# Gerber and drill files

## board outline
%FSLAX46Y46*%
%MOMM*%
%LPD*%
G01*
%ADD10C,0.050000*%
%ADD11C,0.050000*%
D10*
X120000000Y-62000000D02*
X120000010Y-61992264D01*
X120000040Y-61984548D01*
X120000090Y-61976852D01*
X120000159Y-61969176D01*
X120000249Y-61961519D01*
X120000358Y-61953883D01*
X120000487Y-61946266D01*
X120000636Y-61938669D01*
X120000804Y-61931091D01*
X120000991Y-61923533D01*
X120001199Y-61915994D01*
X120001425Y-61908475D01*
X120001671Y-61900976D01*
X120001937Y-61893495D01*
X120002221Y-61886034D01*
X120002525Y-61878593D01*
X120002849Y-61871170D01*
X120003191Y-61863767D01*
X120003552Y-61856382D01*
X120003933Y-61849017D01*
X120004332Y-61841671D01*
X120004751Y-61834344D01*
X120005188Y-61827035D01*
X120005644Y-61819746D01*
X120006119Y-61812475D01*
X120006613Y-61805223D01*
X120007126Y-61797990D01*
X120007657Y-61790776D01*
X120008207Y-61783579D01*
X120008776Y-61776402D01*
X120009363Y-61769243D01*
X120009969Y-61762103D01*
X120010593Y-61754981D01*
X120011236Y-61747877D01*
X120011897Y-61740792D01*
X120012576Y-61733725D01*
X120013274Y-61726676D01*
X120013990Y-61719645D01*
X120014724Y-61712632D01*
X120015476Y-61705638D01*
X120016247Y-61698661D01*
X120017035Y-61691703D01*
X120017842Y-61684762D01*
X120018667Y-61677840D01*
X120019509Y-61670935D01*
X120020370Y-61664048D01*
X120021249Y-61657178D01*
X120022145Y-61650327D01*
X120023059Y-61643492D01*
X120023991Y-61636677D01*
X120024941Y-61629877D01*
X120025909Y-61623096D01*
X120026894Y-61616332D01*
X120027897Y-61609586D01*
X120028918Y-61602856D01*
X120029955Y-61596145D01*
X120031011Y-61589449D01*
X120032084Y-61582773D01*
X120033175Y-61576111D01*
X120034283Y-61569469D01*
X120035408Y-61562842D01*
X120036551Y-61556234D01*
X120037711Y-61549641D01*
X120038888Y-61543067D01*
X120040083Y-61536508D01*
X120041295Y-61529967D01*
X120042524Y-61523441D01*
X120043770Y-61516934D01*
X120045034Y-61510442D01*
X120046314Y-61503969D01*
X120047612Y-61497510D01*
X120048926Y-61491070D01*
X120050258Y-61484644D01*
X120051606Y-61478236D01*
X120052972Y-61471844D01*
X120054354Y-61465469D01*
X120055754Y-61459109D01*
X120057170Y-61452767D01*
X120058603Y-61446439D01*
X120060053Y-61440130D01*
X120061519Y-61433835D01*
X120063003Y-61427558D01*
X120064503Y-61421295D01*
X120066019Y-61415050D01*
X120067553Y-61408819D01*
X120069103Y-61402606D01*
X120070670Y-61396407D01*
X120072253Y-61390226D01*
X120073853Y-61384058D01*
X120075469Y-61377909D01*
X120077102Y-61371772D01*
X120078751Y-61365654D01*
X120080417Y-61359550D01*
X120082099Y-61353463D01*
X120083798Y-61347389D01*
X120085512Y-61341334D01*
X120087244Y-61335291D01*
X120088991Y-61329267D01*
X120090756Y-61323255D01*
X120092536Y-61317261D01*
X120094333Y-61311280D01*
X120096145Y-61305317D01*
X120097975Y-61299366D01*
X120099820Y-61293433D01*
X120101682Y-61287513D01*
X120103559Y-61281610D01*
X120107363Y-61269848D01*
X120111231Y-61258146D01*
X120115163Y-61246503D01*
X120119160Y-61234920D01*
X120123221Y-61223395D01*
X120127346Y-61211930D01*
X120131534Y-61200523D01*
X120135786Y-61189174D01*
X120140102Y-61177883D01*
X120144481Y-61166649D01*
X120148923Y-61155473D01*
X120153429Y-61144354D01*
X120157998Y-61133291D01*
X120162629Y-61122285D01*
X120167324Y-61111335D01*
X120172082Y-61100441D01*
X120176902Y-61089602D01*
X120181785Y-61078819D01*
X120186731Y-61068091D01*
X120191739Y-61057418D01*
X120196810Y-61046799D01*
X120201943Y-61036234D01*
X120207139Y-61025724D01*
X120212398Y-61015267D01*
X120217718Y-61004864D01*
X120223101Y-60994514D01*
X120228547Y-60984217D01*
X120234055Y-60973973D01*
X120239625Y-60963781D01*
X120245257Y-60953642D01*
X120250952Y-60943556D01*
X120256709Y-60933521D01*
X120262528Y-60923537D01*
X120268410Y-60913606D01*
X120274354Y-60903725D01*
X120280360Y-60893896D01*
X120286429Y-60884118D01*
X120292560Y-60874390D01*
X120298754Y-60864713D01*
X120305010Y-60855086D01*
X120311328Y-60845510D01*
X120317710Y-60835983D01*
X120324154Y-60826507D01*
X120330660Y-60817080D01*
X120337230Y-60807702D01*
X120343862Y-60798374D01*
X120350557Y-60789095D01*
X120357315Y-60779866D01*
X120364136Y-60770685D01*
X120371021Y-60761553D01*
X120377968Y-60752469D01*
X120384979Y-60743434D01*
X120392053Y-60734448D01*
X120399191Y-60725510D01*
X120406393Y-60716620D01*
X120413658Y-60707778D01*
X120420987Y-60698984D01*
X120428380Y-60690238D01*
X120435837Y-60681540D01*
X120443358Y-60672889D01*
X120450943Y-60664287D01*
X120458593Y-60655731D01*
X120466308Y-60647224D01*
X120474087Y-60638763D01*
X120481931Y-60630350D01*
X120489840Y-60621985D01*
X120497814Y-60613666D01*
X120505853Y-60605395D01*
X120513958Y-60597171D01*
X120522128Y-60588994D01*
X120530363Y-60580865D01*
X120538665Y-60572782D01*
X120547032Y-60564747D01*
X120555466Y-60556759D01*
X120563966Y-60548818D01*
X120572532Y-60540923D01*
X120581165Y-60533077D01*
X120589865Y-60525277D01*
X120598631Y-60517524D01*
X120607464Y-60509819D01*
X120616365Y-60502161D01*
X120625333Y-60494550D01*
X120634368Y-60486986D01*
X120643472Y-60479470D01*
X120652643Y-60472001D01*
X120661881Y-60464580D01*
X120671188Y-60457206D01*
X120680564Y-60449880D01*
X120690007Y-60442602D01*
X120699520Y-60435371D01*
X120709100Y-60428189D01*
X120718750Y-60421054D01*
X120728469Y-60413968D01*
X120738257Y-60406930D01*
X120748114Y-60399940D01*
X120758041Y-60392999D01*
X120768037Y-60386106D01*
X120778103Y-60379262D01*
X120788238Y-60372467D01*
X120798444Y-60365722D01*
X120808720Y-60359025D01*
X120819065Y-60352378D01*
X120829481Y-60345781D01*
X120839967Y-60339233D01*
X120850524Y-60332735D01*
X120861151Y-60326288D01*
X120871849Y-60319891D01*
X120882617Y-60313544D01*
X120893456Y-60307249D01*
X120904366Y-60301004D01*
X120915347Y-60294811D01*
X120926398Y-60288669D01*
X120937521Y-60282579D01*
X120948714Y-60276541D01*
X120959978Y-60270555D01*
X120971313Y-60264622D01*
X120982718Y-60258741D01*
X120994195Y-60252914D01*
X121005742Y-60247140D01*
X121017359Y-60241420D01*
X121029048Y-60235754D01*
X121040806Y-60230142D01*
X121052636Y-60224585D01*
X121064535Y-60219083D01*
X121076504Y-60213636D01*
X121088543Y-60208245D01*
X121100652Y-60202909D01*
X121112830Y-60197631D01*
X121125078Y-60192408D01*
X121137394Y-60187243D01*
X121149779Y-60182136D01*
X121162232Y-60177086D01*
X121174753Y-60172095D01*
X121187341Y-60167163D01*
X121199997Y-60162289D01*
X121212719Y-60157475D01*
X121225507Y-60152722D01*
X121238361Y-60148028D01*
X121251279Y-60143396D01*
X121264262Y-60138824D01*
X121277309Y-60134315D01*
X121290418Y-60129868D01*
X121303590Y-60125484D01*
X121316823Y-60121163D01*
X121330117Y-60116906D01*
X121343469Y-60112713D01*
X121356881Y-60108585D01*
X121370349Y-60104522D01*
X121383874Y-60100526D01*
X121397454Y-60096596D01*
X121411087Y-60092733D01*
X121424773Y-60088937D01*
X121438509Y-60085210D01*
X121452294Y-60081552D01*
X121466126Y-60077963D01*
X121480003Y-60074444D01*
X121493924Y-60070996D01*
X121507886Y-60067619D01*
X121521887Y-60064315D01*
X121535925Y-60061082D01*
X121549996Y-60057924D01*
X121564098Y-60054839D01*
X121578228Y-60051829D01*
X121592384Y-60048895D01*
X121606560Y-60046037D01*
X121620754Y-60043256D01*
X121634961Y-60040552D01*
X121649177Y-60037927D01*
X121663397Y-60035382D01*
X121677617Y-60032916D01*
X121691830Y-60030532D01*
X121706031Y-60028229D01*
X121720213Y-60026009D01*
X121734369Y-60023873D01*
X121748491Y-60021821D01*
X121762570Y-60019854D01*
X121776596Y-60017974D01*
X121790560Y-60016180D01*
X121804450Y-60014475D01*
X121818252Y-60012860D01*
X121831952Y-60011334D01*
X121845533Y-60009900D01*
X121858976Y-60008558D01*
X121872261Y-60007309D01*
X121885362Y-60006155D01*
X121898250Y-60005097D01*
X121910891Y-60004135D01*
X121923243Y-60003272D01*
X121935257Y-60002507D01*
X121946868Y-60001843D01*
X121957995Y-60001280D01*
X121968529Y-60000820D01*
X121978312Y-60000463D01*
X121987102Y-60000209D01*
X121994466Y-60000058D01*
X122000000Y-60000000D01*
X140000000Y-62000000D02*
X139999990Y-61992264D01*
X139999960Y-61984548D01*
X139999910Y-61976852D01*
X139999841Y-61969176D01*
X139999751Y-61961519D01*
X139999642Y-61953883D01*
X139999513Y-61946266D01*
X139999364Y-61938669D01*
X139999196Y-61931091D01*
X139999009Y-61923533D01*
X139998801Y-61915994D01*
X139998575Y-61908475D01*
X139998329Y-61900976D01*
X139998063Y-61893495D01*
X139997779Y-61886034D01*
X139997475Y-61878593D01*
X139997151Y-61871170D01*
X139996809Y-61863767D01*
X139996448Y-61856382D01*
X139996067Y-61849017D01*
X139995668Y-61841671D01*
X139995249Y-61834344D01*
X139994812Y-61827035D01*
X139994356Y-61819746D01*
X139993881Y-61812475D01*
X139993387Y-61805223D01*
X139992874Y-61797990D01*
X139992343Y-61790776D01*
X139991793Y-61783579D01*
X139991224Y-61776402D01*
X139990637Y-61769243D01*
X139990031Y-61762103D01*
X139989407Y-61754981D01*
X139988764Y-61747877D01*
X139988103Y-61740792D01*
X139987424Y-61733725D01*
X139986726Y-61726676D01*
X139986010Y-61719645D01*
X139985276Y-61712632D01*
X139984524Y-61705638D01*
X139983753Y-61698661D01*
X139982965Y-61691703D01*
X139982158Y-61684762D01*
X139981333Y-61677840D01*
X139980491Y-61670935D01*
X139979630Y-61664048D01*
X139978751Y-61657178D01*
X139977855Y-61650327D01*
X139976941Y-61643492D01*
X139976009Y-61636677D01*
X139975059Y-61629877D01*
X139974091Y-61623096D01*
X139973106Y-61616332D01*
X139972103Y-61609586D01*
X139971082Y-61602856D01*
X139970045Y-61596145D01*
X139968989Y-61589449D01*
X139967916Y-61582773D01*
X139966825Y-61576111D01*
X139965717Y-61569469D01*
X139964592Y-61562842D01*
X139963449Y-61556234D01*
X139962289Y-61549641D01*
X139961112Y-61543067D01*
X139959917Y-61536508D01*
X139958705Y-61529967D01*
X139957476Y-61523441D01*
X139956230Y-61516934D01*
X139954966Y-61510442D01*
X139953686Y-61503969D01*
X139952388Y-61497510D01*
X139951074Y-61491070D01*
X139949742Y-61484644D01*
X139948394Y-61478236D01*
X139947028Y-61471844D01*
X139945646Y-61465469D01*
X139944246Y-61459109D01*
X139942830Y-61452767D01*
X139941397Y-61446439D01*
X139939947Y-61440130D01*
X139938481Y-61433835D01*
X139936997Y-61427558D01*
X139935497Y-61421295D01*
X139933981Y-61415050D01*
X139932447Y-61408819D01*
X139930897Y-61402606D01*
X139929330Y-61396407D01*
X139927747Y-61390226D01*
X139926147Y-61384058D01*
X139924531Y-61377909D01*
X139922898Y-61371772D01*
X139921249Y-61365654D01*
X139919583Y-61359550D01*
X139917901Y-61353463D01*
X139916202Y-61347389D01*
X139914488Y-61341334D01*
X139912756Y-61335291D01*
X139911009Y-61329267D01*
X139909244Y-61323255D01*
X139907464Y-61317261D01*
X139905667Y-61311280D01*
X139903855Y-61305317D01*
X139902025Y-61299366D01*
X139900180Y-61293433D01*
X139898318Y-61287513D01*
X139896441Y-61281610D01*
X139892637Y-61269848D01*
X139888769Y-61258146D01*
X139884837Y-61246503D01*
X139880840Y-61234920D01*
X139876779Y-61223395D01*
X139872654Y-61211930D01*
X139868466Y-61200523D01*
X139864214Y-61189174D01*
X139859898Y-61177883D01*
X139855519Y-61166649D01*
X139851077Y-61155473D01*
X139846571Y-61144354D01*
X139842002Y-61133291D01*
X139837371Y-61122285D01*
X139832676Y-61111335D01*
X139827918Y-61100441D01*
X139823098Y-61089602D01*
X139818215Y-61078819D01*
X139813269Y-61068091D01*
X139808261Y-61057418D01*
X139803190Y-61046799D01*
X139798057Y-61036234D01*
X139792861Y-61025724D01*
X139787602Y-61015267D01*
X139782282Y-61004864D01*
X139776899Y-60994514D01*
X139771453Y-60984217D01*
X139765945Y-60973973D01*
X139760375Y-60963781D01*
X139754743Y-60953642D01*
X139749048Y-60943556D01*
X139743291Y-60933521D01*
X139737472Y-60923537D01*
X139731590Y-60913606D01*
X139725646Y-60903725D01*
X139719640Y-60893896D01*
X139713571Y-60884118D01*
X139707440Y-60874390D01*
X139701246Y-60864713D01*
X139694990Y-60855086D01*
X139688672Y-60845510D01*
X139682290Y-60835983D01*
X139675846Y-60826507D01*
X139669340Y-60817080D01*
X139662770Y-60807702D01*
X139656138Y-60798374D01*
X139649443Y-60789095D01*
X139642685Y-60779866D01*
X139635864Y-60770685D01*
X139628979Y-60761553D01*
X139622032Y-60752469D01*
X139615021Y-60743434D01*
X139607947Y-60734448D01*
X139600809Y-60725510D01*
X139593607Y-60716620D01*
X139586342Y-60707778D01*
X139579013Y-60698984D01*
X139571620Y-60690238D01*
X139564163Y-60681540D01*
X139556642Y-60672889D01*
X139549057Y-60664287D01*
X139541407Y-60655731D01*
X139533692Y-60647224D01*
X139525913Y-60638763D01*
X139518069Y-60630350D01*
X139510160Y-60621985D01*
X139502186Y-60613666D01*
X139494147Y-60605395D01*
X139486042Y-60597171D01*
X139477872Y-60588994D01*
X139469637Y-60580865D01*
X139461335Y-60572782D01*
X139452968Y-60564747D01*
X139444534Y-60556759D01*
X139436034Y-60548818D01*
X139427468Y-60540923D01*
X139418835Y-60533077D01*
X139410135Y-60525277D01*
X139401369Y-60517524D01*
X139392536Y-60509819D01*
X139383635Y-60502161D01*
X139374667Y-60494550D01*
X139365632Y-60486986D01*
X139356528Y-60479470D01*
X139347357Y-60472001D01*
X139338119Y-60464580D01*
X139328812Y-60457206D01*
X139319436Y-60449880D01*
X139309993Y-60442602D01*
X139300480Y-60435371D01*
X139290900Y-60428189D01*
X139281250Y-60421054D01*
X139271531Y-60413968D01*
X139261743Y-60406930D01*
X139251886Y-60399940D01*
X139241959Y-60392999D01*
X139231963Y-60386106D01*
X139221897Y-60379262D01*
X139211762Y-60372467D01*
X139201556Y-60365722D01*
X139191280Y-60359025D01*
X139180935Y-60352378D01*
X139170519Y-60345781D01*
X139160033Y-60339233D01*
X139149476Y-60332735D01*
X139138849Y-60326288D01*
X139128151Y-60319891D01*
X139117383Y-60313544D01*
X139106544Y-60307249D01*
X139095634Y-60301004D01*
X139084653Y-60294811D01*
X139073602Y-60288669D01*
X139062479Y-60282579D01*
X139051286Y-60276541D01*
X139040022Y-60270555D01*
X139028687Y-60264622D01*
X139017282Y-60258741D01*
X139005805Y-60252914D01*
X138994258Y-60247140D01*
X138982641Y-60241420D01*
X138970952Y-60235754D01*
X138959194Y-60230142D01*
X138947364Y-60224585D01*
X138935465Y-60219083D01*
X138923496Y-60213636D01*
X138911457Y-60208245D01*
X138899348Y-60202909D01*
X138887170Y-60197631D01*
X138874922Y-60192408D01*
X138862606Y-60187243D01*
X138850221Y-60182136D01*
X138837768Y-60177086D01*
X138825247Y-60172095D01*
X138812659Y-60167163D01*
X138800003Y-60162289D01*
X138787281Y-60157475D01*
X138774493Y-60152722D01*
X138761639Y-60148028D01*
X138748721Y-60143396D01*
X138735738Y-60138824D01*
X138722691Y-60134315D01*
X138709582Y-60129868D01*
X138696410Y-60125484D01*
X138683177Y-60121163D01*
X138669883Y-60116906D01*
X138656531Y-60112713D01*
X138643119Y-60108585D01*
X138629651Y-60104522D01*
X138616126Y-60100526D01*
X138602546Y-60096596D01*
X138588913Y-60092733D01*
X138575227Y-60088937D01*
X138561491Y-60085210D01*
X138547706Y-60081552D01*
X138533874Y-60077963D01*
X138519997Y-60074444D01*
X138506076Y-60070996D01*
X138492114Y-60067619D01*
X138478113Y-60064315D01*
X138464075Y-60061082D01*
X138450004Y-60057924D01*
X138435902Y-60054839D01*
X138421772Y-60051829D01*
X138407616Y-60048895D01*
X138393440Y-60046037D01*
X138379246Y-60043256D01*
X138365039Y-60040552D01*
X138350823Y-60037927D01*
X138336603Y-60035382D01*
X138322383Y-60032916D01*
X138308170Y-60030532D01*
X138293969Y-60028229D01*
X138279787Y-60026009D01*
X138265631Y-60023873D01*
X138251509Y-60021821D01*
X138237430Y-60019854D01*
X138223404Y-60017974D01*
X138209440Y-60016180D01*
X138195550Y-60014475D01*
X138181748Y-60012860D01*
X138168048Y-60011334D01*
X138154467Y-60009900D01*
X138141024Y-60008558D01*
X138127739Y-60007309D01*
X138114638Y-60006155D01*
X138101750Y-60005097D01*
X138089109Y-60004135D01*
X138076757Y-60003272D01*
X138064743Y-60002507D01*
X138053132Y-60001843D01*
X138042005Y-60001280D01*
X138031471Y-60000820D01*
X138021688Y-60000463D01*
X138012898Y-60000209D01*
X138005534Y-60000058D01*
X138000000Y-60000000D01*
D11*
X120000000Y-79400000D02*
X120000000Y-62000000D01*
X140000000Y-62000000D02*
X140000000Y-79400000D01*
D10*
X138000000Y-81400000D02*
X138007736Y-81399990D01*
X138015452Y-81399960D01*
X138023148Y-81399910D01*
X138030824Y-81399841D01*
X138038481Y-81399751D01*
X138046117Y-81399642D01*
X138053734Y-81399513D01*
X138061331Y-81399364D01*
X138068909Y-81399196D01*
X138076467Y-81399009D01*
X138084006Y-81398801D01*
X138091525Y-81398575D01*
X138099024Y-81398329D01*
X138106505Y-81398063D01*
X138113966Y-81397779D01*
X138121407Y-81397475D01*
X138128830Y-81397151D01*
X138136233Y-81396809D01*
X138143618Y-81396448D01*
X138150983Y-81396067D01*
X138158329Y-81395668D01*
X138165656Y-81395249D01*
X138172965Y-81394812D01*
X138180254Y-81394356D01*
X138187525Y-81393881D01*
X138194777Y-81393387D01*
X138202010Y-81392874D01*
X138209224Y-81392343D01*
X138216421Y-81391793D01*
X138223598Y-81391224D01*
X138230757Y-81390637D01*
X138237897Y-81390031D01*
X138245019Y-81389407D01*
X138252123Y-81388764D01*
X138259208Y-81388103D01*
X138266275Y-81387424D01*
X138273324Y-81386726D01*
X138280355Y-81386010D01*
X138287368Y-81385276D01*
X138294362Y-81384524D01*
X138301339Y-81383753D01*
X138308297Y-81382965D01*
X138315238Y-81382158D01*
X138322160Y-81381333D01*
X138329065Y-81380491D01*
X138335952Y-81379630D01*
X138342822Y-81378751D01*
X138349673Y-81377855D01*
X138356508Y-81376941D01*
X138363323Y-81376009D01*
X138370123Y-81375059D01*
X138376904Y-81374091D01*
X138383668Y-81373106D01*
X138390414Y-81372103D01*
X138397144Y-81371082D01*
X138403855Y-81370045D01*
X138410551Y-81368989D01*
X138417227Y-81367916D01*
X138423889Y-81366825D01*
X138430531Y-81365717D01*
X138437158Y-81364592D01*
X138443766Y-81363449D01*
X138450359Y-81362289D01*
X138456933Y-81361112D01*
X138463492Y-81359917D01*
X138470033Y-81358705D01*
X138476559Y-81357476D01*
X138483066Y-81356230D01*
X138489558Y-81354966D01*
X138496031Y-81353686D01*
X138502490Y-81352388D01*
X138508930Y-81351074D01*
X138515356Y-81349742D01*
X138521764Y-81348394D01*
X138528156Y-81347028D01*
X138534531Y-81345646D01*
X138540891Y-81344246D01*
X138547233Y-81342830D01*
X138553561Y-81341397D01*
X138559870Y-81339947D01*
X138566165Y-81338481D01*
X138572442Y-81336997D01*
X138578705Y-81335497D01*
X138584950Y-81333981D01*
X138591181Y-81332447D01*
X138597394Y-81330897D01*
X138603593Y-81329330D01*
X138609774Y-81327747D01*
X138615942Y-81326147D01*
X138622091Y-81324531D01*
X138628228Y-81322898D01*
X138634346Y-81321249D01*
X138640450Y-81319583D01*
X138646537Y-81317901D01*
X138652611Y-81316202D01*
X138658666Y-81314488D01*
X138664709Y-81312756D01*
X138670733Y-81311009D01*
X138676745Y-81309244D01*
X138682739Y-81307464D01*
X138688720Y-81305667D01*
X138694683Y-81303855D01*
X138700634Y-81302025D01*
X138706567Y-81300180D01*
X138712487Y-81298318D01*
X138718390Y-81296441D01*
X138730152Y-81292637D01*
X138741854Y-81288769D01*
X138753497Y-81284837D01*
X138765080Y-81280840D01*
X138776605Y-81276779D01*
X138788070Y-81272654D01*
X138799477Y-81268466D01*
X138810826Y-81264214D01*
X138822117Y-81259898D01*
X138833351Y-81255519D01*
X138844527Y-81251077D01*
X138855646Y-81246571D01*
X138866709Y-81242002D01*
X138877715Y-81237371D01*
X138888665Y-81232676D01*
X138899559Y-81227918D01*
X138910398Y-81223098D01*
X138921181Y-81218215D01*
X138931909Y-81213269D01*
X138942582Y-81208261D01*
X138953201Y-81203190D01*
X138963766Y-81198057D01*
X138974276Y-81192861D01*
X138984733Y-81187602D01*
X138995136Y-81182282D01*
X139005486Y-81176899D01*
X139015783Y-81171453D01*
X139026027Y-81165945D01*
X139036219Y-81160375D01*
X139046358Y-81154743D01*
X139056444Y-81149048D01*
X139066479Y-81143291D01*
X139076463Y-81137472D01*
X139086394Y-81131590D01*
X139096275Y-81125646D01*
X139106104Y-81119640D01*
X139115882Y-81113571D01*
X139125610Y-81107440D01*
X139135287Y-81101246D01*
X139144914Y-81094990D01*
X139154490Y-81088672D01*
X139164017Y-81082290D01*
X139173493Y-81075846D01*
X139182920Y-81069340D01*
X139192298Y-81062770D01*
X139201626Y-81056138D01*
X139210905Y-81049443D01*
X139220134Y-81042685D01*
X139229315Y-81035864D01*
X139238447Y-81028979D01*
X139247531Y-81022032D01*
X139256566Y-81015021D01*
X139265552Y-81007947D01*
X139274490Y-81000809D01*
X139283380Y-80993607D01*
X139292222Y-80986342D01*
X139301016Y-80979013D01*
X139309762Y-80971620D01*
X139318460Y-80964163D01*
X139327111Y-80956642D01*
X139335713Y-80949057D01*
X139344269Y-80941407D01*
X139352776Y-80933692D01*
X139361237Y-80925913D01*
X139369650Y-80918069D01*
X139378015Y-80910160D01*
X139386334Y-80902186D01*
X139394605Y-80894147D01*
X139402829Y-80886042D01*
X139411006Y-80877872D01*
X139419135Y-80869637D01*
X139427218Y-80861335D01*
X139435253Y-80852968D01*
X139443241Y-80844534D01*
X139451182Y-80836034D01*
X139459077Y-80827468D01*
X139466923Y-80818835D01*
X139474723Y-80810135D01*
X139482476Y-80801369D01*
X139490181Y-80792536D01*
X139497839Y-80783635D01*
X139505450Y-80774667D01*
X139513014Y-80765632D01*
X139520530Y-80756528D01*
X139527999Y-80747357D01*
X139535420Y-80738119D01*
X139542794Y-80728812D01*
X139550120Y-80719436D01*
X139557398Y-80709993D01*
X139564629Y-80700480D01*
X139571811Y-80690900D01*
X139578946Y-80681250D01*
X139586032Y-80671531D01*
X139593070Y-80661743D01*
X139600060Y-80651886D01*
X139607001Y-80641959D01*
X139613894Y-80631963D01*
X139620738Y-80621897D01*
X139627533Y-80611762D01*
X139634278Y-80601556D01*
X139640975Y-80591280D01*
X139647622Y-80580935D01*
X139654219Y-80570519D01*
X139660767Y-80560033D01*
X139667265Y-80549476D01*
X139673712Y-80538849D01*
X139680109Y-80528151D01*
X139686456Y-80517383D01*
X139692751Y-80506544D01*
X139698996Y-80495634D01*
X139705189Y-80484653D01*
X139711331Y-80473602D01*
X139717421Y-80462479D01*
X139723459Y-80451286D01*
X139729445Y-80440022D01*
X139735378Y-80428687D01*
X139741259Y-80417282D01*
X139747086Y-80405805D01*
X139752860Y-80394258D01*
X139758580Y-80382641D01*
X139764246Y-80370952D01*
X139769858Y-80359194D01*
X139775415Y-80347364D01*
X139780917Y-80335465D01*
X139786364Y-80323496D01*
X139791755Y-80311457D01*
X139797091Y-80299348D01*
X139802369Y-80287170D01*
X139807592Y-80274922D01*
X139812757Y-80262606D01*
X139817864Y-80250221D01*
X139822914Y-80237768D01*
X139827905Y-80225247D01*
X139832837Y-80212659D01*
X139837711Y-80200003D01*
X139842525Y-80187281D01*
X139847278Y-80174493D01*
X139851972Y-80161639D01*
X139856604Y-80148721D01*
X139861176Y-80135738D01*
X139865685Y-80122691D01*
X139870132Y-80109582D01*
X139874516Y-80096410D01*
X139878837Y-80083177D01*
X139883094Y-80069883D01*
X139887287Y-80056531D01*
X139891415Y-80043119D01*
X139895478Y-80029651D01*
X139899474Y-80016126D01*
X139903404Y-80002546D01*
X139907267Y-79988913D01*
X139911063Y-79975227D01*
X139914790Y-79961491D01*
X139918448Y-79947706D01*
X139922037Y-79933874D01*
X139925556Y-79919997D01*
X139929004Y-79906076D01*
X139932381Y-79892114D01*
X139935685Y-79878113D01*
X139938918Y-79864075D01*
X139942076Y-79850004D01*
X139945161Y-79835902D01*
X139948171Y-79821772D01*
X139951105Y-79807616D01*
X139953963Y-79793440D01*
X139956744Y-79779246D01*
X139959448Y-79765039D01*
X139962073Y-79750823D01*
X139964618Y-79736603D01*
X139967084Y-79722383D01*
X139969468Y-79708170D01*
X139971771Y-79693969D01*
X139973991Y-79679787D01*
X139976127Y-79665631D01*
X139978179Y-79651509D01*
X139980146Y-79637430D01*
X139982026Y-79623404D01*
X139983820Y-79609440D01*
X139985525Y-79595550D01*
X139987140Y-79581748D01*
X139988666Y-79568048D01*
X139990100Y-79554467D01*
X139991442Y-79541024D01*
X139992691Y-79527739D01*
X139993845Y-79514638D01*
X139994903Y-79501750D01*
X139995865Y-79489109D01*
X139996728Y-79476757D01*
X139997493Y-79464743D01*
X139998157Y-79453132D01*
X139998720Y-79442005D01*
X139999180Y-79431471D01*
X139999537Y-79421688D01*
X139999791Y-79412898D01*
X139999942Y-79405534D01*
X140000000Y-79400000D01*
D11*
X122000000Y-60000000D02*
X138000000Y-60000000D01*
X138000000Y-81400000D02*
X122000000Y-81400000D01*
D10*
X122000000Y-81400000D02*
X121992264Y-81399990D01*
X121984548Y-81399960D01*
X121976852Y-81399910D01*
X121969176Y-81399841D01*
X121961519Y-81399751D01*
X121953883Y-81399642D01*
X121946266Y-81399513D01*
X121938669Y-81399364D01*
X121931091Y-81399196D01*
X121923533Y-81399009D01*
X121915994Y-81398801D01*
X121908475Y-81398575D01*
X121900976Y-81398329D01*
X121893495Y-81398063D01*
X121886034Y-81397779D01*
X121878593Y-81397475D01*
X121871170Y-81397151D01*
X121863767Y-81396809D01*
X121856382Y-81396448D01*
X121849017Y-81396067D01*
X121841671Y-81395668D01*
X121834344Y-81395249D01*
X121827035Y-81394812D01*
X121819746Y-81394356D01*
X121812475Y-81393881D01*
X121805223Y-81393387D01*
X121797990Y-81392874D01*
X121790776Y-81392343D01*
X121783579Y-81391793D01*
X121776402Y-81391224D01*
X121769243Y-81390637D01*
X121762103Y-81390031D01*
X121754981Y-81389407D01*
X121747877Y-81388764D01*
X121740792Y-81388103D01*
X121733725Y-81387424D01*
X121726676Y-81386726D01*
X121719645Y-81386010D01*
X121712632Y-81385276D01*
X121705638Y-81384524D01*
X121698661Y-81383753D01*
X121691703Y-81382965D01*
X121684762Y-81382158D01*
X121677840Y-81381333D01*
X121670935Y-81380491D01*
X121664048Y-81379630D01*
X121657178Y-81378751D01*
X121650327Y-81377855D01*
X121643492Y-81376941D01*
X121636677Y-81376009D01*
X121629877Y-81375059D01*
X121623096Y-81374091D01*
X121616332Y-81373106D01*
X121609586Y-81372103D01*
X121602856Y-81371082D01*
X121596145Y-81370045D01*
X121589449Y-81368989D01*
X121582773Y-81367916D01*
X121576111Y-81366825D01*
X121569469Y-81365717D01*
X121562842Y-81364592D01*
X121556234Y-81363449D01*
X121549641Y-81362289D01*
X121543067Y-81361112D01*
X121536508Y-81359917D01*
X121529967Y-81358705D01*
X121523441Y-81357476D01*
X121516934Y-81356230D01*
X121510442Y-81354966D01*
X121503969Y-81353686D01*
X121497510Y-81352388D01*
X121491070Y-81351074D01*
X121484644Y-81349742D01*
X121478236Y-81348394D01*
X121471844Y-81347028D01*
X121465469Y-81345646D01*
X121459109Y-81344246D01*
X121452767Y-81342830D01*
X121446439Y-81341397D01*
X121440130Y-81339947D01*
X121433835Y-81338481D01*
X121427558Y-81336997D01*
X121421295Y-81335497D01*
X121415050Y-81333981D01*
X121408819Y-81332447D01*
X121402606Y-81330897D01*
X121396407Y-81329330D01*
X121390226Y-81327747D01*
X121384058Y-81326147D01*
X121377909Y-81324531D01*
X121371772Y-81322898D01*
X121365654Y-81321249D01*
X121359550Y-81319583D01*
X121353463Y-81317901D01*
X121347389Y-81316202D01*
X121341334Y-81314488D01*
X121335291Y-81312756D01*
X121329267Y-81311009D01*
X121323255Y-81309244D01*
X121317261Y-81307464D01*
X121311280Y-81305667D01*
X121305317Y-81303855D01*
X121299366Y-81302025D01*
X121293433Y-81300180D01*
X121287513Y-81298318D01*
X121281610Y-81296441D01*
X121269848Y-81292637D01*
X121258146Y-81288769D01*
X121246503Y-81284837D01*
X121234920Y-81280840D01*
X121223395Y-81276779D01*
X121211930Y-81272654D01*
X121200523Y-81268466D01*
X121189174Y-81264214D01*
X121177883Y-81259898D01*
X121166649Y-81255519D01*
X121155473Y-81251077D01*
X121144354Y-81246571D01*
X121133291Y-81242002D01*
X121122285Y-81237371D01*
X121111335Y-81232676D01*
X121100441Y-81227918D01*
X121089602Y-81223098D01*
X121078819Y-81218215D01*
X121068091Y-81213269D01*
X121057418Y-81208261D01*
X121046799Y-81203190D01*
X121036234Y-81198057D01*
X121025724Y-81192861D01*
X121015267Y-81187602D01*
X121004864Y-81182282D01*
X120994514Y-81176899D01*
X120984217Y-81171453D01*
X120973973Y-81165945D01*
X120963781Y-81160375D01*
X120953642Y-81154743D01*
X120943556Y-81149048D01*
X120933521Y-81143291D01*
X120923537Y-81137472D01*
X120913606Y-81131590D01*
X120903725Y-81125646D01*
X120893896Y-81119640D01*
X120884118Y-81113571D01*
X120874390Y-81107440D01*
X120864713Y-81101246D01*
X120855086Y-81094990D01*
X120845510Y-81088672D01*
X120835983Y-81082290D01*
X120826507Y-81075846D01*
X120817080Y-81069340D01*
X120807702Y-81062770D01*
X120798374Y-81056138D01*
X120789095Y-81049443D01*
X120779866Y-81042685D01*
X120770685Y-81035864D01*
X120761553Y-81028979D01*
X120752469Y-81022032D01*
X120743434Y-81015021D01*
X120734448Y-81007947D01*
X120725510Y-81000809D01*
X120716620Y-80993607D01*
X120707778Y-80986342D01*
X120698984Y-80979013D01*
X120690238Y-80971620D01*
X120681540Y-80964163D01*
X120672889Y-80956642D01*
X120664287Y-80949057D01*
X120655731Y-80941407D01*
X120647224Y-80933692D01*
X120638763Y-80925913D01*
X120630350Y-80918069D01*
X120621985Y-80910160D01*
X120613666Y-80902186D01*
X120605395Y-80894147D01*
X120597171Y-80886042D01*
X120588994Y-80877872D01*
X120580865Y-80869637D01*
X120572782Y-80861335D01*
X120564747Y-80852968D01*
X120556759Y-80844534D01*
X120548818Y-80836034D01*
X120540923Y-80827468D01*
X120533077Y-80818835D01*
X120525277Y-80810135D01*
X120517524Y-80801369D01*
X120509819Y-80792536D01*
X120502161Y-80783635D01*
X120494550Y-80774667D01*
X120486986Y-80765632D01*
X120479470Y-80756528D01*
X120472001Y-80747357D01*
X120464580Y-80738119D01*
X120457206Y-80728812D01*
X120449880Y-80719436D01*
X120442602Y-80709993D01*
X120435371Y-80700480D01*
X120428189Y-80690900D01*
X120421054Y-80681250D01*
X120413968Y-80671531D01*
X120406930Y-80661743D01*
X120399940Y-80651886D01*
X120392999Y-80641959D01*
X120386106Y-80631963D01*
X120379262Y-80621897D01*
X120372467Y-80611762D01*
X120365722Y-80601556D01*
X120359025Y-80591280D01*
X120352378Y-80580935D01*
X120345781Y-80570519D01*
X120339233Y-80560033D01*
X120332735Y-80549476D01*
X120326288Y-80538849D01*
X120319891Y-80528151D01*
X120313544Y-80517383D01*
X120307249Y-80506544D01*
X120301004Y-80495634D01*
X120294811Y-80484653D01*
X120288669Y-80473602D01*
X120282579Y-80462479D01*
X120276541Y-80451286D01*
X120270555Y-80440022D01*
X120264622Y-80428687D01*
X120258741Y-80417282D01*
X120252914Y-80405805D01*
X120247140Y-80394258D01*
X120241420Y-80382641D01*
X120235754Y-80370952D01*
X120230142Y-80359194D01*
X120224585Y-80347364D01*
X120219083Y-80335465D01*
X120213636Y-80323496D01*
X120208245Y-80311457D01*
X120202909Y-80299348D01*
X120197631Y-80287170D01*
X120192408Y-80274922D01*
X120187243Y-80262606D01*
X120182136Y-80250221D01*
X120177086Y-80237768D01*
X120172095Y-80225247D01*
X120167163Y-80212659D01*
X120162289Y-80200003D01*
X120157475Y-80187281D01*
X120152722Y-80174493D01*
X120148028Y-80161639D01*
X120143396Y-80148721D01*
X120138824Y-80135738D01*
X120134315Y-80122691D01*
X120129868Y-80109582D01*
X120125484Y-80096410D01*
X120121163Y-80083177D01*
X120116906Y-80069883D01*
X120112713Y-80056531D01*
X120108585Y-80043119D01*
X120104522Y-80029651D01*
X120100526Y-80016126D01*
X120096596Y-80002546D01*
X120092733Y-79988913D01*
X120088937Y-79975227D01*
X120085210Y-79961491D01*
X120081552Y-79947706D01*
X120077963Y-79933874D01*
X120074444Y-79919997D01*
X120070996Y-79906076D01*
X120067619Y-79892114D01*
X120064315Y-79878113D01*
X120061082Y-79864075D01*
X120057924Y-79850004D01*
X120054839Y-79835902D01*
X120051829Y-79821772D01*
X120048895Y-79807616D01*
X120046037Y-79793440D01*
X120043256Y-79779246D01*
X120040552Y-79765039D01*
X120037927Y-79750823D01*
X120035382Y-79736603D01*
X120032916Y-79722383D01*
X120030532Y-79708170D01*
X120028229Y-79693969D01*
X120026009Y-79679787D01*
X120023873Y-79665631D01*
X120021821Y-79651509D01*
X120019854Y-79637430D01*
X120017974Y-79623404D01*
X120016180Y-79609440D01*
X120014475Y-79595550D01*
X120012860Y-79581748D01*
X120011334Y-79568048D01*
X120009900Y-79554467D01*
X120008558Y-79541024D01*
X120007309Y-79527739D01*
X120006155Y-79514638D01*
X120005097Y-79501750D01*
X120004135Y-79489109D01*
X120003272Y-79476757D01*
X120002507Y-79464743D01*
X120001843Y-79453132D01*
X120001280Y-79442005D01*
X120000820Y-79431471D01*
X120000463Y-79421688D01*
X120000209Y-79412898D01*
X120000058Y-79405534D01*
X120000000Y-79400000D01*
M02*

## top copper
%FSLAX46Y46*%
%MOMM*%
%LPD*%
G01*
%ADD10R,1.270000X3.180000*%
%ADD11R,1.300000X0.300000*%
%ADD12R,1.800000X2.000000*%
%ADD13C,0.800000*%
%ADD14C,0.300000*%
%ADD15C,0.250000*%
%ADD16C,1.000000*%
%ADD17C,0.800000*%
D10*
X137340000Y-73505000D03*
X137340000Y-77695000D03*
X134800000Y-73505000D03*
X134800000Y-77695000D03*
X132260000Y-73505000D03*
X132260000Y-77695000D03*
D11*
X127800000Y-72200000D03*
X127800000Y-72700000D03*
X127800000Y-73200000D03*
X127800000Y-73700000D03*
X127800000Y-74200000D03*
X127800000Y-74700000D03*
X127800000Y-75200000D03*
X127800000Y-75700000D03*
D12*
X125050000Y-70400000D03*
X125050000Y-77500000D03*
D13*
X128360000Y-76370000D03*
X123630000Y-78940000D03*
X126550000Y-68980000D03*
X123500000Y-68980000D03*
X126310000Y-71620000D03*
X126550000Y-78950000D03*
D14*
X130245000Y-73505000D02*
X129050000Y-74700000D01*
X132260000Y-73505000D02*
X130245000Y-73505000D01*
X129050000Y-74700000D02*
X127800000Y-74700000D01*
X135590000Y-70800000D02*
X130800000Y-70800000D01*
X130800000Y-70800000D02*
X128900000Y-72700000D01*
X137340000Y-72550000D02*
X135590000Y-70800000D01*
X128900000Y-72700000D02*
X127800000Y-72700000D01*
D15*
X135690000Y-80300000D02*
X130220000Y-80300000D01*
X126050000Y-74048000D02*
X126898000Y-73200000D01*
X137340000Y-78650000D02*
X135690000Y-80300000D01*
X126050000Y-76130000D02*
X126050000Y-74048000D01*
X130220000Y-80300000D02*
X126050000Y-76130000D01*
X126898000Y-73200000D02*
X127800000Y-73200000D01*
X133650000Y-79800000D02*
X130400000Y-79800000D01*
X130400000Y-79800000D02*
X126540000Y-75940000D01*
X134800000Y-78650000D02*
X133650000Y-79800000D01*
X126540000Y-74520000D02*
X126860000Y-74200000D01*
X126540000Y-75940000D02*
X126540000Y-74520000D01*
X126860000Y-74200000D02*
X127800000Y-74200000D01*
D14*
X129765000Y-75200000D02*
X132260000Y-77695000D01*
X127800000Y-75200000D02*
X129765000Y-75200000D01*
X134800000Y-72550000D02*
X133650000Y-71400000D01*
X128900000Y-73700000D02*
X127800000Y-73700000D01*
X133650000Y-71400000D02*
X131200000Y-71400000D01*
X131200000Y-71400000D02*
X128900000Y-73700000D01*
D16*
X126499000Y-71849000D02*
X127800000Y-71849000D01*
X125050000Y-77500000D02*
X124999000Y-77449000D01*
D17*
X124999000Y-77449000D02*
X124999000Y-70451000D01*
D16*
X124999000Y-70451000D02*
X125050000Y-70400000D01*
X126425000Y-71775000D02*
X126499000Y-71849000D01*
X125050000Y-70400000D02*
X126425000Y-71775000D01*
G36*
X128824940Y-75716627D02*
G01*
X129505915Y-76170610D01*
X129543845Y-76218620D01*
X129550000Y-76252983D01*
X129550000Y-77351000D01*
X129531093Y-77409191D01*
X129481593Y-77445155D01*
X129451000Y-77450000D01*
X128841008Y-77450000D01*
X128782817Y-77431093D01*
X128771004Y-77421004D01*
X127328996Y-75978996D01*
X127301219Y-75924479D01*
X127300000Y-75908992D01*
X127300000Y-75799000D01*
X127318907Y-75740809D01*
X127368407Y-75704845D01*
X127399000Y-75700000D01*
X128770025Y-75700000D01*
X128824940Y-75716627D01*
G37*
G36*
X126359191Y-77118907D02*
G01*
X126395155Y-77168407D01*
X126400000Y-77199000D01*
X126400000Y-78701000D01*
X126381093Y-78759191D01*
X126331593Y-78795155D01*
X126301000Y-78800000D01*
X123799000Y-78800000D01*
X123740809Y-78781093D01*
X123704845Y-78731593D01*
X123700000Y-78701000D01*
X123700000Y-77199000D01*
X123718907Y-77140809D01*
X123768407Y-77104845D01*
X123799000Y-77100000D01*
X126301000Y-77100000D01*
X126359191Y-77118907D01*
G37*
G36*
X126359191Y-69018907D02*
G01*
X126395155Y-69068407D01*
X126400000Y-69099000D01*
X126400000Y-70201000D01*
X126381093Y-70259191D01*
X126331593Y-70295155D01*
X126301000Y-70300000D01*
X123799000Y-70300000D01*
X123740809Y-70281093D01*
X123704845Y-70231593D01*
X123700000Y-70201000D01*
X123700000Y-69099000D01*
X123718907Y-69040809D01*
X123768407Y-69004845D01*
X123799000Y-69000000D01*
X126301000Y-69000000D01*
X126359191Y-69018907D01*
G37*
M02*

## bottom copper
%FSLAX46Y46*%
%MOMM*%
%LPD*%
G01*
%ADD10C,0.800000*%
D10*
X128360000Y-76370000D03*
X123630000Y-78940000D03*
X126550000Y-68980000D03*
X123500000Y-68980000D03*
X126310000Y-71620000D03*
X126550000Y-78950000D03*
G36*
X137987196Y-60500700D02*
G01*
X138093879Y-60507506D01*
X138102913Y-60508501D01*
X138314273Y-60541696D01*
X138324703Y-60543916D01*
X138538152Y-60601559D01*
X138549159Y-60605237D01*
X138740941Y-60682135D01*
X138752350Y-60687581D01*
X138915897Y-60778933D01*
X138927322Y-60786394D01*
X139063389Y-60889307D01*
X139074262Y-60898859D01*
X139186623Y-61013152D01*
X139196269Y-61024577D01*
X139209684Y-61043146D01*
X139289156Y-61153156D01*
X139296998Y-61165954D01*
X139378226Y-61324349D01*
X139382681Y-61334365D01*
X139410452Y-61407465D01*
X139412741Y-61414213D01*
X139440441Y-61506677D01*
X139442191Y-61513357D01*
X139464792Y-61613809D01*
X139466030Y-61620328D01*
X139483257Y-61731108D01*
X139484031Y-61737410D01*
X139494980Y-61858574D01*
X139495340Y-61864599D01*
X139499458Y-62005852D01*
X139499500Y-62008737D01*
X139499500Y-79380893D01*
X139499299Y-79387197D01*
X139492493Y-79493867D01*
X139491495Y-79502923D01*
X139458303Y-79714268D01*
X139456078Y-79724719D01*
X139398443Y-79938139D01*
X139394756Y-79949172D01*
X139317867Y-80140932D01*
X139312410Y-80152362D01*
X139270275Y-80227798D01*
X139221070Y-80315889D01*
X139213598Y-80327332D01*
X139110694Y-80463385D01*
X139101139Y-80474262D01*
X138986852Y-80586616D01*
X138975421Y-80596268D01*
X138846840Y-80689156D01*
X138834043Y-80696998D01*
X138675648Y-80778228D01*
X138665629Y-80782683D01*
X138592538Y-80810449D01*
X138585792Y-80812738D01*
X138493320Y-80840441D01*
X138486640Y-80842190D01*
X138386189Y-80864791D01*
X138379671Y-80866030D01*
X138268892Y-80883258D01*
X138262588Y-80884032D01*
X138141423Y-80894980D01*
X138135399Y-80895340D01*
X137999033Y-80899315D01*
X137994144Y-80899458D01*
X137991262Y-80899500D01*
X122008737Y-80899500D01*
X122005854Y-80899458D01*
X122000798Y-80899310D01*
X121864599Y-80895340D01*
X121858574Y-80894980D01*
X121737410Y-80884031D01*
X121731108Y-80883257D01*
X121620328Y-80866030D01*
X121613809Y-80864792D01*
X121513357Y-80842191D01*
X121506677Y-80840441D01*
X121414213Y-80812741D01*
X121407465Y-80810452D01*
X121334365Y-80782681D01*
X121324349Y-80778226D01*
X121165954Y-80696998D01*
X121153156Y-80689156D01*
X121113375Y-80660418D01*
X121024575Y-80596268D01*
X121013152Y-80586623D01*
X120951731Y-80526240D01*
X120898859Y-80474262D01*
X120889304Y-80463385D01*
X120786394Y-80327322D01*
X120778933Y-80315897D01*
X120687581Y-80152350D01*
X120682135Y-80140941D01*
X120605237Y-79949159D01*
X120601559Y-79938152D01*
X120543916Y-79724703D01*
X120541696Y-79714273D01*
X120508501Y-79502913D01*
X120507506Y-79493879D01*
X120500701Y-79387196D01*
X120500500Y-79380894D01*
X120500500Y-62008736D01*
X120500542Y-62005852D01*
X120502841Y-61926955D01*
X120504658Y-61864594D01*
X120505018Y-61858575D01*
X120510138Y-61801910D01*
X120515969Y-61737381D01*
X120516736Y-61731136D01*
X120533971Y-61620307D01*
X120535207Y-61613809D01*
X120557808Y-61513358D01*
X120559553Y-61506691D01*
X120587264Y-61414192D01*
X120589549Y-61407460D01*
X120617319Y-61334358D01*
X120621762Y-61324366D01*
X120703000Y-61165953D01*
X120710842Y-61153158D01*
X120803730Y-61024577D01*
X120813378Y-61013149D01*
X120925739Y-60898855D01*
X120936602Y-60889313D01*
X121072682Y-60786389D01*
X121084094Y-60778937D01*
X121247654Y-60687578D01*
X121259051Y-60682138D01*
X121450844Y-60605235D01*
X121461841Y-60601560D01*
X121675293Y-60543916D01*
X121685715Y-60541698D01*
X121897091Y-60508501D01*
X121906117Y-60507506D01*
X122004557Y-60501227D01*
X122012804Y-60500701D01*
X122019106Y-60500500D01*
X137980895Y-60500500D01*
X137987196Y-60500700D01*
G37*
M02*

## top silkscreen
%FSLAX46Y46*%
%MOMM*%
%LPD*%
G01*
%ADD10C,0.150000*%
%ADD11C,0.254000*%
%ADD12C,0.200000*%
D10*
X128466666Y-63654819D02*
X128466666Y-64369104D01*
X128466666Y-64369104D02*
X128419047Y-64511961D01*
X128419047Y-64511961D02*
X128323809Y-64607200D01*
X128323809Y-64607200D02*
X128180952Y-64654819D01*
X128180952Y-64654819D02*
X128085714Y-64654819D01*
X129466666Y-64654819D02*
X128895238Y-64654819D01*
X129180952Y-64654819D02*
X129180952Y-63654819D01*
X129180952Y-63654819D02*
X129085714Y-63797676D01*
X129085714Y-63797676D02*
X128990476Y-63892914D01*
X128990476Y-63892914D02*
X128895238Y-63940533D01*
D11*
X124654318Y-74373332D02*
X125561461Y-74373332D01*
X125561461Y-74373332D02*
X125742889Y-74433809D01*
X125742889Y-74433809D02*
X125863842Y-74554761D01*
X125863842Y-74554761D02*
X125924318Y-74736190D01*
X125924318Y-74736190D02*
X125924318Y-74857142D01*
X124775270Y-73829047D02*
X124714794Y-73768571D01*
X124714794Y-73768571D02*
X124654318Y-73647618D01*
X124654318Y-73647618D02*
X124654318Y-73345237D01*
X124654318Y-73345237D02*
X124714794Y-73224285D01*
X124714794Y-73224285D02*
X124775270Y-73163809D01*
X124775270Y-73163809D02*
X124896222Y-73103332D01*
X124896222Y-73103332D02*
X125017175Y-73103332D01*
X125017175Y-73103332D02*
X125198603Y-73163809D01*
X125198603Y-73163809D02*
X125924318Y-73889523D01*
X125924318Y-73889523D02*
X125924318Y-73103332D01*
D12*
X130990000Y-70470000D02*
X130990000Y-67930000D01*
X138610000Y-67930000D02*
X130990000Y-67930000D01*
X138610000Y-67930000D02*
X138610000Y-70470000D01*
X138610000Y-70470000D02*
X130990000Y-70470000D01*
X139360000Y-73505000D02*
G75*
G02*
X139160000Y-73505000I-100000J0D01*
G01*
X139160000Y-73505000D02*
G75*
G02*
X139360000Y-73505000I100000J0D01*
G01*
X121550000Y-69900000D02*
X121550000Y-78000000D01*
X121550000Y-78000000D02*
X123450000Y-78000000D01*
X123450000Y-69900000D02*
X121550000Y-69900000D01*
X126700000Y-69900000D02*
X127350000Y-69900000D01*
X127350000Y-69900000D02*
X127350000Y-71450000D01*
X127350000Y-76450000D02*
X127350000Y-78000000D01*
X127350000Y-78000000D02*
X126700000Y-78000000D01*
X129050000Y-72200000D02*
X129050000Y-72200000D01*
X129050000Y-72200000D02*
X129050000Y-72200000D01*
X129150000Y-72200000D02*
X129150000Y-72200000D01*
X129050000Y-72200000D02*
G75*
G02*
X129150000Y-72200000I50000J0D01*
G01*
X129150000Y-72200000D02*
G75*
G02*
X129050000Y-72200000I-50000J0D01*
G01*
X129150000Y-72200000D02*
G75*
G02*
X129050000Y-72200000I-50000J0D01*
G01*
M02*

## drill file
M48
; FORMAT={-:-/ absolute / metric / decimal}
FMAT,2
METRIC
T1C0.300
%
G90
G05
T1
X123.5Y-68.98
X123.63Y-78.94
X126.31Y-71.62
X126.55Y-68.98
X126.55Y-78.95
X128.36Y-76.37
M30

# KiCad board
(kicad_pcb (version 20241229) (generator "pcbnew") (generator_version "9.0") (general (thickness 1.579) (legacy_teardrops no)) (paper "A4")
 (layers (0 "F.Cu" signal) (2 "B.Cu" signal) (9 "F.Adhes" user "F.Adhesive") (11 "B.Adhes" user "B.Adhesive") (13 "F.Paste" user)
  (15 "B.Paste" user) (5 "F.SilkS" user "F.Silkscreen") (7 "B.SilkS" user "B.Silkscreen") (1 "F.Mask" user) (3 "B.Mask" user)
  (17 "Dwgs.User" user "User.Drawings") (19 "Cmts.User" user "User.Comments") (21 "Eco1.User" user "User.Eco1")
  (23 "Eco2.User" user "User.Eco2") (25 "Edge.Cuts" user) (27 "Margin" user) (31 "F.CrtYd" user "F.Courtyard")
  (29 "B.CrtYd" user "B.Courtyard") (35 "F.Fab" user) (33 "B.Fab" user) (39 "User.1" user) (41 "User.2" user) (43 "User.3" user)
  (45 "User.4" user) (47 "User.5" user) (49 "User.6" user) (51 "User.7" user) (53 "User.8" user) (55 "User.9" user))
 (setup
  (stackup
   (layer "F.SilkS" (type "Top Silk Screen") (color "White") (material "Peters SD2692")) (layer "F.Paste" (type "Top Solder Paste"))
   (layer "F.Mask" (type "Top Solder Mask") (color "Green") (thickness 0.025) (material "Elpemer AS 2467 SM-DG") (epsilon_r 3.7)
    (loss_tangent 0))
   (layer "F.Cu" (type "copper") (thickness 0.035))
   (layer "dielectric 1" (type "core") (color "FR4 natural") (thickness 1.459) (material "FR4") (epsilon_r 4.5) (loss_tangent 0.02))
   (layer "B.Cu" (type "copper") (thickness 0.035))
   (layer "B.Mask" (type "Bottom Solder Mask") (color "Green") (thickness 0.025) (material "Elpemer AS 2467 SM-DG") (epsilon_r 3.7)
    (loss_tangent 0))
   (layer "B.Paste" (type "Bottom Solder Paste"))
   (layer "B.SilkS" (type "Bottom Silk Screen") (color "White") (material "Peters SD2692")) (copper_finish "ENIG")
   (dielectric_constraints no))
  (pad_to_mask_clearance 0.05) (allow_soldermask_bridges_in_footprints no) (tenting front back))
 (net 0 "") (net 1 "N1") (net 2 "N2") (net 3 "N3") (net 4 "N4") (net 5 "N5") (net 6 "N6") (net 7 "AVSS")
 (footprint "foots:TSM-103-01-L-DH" (layer "F.Cu") (at 134.8 69.2)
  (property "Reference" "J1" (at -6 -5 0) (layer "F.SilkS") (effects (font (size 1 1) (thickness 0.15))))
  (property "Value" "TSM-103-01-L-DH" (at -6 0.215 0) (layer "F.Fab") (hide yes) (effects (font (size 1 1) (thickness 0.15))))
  (fp_line (start -3.81 1.27) (end -3.81 -1.27) (stroke (width 0.2) (type solid)) (layer "F.SilkS"))
  (fp_line (start 3.81 -1.27) (end -3.81 -1.27) (stroke (width 0.2) (type solid)) (layer "F.SilkS"))
  (fp_line (start 3.81 -1.27) (end 3.81 1.27) (stroke (width 0.2) (type solid)) (layer "F.SilkS"))
  (fp_line (start 3.81 1.27) (end -3.81 1.27) (stroke (width 0.2) (type solid)) (layer "F.SilkS"))
  (fp_circle (center 4.46 4.305) (end 4.56 4.305) (stroke (width 0.2) (type solid)) (fill no) (layer "F.SilkS"))
  (pad "01" smd rect (at 2.54 4.305) (size 1.27 3.18) (layers "F.Cu" "F.Mask" "F.Paste") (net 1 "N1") (solder_mask_margin 0.102))
  (pad "02" smd rect (at 2.54 8.495) (size 1.27 3.18) (layers "F.Cu" "F.Mask" "F.Paste") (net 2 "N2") (solder_mask_margin 0.102))
  (pad "03" smd rect (at 0 4.305) (size 1.27 3.18) (layers "F.Cu" "F.Mask" "F.Paste") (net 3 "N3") (solder_mask_margin 0.102))
  (pad "04" smd rect (at 0 8.495) (size 1.27 3.18) (layers "F.Cu" "F.Mask" "F.Paste") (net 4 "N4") (solder_mask_margin 0.102))
  (pad "05" smd rect (at -2.54 4.305) (size 1.27 3.18) (layers "F.Cu" "F.Mask" "F.Paste") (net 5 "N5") (solder_mask_margin 0.102))
  (pad "06" smd rect (at -2.54 8.495) (size 1.27 3.18) (layers "F.Cu" "F.Mask" "F.Paste") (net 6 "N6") (solder_mask_margin 0.102)))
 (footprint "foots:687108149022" (layer "F.Cu") (at 125.05 73.95 -90)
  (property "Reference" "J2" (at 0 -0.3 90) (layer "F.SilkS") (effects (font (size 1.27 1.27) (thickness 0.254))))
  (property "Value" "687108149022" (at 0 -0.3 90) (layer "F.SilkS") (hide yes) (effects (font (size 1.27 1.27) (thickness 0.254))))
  (fp_line (start -4.05 3.5) (end 4.05 3.5) (stroke (width 0.2) (type solid)) (layer "F.SilkS"))
  (fp_line (start 4.05 3.5) (end 4.05 1.6) (stroke (width 0.2) (type solid)) (layer "F.SilkS"))
  (fp_line (start -4.05 1.6) (end -4.05 3.5) (stroke (width 0.2) (type solid)) (layer "F.SilkS"))
  (fp_line (start -4.05 -1.65) (end -4.05 -2.3) (stroke (width 0.2) (type solid)) (layer "F.SilkS"))
  (fp_line (start -4.05 -2.3) (end -2.5 -2.3) (stroke (width 0.2) (type solid)) (layer "F.SilkS"))
  (fp_line (start 2.5 -2.3) (end 4.05 -2.3) (stroke (width 0.2) (type solid)) (layer "F.SilkS"))
  (fp_line (start 4.05 -2.3) (end 4.05 -1.65) (stroke (width 0.2) (type solid)) (layer "F.SilkS"))
  (fp_line (start -1.75 -4) (end -1.75 -4) (stroke (width 0.2) (type solid)) (layer "F.SilkS"))
  (fp_line (start -1.75 -4) (end -1.75 -4) (stroke (width 0.2) (type solid)) (layer "F.SilkS"))
  (fp_line (start -1.75 -4.1) (end -1.75 -4.1) (stroke (width 0.2) (type solid)) (layer "F.SilkS"))
  (fp_arc (start -1.75 -4) (mid -1.8 -4.05) (end -1.75 -4.1) (stroke (width 0.2) (type solid)) (layer "F.SilkS"))
  (fp_arc (start -1.75 -4.1) (mid -1.7 -4.05) (end -1.75 -4) (stroke (width 0.2) (type solid)) (layer "F.SilkS"))
  (fp_arc (start -1.75 -4.1) (mid -1.7 -4.05) (end -1.75 -4) (stroke (width 0.2) (type solid)) (layer "F.SilkS"))
  (pad "1" smd rect (at -1.75 -2.75 270) (size 0.3 1.3) (layers "F.Cu" "F.Mask" "F.Paste") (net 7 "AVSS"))
  (pad "2" smd rect (at -1.25 -2.75 270) (size 0.3 1.3) (layers "F.Cu" "F.Mask" "F.Paste") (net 1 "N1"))
  (pad "3" smd rect (at -0.75 -2.75 270) (size 0.3 1.3) (layers "F.Cu" "F.Mask" "F.Paste") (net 2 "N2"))
  (pad "4" smd rect (at -0.25 -2.75 270) (size 0.3 1.3) (layers "F.Cu" "F.Mask" "F.Paste") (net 3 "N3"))
  (pad "5" smd rect (at 0.25 -2.75 270) (size 0.3 1.3) (layers "F.Cu" "F.Mask" "F.Paste") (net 4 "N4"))
  (pad "6" smd rect (at 0.75 -2.75 270) (size 0.3 1.3) (layers "F.Cu" "F.Mask" "F.Paste") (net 5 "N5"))
  (pad "7" smd rect (at 1.25 -2.75 270) (size 0.3 1.3) (layers "F.Cu" "F.Mask" "F.Paste") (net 6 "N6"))
  (pad "8" smd rect (at 1.75 -2.75 270) (size 0.3 1.3) (layers "F.Cu" "F.Mask" "F.Paste") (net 7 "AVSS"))
  (pad "MP1" smd rect (at -3.55 0) (size 1.8 2) (layers "F.Cu" "F.Mask" "F.Paste") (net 7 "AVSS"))
  (pad "MP2" smd rect (at 3.55 0) (size 1.8 2) (layers "F.Cu" "F.Mask" "F.Paste") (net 7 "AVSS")))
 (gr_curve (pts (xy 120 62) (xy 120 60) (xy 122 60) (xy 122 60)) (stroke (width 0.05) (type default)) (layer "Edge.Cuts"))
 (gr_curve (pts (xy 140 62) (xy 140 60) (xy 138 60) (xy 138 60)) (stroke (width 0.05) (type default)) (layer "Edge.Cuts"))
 (gr_line (start 120 79.4) (end 120 62) (stroke (width 0.05) (type default)) (layer "Edge.Cuts"))
 (gr_line (start 140 62) (end 140 79.4) (stroke (width 0.05) (type default)) (layer "Edge.Cuts"))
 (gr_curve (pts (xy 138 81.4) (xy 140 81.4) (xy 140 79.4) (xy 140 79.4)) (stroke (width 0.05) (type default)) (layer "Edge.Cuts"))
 (gr_line (start 122 60) (end 138 60) (stroke (width 0.05) (type default)) (layer "Edge.Cuts"))
 (gr_line (start 138 81.4) (end 122 81.4) (stroke (width 0.05) (type default)) (layer "Edge.Cuts"))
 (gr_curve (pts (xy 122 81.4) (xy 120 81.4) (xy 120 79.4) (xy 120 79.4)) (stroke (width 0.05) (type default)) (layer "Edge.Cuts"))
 (segment (start 130.245 73.505) (end 129.05 74.7) (width 0.3) (layer "F.Cu") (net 5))
 (segment (start 132.26 73.505) (end 130.245 73.505) (width 0.3) (layer "F.Cu") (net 5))
 (segment (start 129.05 74.7) (end 127.8 74.7) (width 0.3) (layer "F.Cu") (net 5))
 (segment (start 135.59 70.8) (end 130.8 70.8) (width 0.3) (layer "F.Cu") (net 1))
 (segment (start 130.8 70.8) (end 128.9 72.7) (width 0.3) (layer "F.Cu") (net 1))
 (segment (start 137.34 72.55) (end 135.59 70.8) (width 0.3) (layer "F.Cu") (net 1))
 (segment (start 128.9 72.7) (end 127.8 72.7) (width 0.3) (layer "F.Cu") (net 1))
 (segment (start 135.69 80.3) (end 130.22 80.3) (width 0.25) (layer "F.Cu") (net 2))
 (segment (start 126.05 74.048) (end 126.898 73.2) (width 0.25) (layer "F.Cu") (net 2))
 (segment (start 137.34 78.65) (end 135.69 80.3) (width 0.25) (layer "F.Cu") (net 2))
 (segment (start 126.05 76.13) (end 126.05 74.048) (width 0.25) (layer "F.Cu") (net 2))
 (segment (start 130.22 80.3) (end 126.05 76.13) (width 0.25) (layer "F.Cu") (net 2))
 (segment (start 126.898 73.2) (end 127.8 73.2) (width 0.25) (layer "F.Cu") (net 2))
 (segment (start 133.65 79.8) (end 130.4 79.8) (width 0.25) (layer "F.Cu") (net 4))
 (segment (start 130.4 79.8) (end 126.54 75.94) (width 0.25) (layer "F.Cu") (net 4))
 (segment (start 134.8 78.65) (end 133.65 79.8) (width 0.25) (layer "F.Cu") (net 4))
 (segment (start 126.54 74.52) (end 126.86 74.2) (width 0.25) (layer "F.Cu") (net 4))
 (segment (start 126.54 75.94) (end 126.54 74.52) (width 0.25) (layer "F.Cu") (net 4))
 (segment (start 126.86 74.2) (end 127.8 74.2) (width 0.25) (layer "F.Cu") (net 4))
 (segment (start 129.765 75.2) (end 132.26 77.695) (width 0.3) (layer "F.Cu") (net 6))
 (segment (start 127.8 75.2) (end 129.765 75.2) (width 0.3) (layer "F.Cu") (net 6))
 (segment (start 134.8 72.55) (end 133.65 71.4) (width 0.3) (layer "F.Cu") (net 3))
 (segment (start 128.9 73.7) (end 127.8 73.7) (width 0.3) (layer "F.Cu") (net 3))
 (segment (start 133.65 71.4) (end 131.2 71.4) (width 0.3) (layer "F.Cu") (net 3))
 (segment (start 131.2 71.4) (end 128.9 73.7) (width 0.3) (layer "F.Cu") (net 3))
 (segment (start 126.499 71.849) (end 127.8 71.849) (width 1) (layer "F.Cu") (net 7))
 (segment (start 125.05 77.5) (end 124.999 77.449) (width 1) (layer "F.Cu") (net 7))
 (segment (start 124.999 77.449) (end 124.999 70.451) (width 0.8) (layer "F.Cu") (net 7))
 (segment (start 124.999 70.451) (end 125.05 70.4) (width 1) (layer "F.Cu") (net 7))
 (segment (start 126.425 71.775) (end 126.499 71.849) (width 1) (layer "F.Cu") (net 7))
 (segment (start 125.05 70.4) (end 126.425 71.775) (width 1) (layer "F.Cu") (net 7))
 (via (at 128.36 76.37) (size 0.8) (drill 0.3) (layers "F.Cu" "B.Cu") (free yes) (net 7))
 (via (at 123.63 78.94) (size 0.8) (drill 0.3) (layers "F.Cu" "B.Cu") (free yes) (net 7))
 (via (at 126.55 68.98) (size 0.8) (drill 0.3) (layers "F.Cu" "B.Cu") (free yes) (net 7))
 (via (at 123.5 68.98) (size 0.8) (drill 0.3) (layers "F.Cu" "B.Cu") (free yes) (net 7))
 (via (at 126.31 71.62) (size 0.8) (drill 0.3) (layers "F.Cu" "B.Cu") (free yes) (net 7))
 (via (at 126.55 78.95) (size 0.8) (drill 0.3) (layers "F.Cu" "B.Cu") (free yes) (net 7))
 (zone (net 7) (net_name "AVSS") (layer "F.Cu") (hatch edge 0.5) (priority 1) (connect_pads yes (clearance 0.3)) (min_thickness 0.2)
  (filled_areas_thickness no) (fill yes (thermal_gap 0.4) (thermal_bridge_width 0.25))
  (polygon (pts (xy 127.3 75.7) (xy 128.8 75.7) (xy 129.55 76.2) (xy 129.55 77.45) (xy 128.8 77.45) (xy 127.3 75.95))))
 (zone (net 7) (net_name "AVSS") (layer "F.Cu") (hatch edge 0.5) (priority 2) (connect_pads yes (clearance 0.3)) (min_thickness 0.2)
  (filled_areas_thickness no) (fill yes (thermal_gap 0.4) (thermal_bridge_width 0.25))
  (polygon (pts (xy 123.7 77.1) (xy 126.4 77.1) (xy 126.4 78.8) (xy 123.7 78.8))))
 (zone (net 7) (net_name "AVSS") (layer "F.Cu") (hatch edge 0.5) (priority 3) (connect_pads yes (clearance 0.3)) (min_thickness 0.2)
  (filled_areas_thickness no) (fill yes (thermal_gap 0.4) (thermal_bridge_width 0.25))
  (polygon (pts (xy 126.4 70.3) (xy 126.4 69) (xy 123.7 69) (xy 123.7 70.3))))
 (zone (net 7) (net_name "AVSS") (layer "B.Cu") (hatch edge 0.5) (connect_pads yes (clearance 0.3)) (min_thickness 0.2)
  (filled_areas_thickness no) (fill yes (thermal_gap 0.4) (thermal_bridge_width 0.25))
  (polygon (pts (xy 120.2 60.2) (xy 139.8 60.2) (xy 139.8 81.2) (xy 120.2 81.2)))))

